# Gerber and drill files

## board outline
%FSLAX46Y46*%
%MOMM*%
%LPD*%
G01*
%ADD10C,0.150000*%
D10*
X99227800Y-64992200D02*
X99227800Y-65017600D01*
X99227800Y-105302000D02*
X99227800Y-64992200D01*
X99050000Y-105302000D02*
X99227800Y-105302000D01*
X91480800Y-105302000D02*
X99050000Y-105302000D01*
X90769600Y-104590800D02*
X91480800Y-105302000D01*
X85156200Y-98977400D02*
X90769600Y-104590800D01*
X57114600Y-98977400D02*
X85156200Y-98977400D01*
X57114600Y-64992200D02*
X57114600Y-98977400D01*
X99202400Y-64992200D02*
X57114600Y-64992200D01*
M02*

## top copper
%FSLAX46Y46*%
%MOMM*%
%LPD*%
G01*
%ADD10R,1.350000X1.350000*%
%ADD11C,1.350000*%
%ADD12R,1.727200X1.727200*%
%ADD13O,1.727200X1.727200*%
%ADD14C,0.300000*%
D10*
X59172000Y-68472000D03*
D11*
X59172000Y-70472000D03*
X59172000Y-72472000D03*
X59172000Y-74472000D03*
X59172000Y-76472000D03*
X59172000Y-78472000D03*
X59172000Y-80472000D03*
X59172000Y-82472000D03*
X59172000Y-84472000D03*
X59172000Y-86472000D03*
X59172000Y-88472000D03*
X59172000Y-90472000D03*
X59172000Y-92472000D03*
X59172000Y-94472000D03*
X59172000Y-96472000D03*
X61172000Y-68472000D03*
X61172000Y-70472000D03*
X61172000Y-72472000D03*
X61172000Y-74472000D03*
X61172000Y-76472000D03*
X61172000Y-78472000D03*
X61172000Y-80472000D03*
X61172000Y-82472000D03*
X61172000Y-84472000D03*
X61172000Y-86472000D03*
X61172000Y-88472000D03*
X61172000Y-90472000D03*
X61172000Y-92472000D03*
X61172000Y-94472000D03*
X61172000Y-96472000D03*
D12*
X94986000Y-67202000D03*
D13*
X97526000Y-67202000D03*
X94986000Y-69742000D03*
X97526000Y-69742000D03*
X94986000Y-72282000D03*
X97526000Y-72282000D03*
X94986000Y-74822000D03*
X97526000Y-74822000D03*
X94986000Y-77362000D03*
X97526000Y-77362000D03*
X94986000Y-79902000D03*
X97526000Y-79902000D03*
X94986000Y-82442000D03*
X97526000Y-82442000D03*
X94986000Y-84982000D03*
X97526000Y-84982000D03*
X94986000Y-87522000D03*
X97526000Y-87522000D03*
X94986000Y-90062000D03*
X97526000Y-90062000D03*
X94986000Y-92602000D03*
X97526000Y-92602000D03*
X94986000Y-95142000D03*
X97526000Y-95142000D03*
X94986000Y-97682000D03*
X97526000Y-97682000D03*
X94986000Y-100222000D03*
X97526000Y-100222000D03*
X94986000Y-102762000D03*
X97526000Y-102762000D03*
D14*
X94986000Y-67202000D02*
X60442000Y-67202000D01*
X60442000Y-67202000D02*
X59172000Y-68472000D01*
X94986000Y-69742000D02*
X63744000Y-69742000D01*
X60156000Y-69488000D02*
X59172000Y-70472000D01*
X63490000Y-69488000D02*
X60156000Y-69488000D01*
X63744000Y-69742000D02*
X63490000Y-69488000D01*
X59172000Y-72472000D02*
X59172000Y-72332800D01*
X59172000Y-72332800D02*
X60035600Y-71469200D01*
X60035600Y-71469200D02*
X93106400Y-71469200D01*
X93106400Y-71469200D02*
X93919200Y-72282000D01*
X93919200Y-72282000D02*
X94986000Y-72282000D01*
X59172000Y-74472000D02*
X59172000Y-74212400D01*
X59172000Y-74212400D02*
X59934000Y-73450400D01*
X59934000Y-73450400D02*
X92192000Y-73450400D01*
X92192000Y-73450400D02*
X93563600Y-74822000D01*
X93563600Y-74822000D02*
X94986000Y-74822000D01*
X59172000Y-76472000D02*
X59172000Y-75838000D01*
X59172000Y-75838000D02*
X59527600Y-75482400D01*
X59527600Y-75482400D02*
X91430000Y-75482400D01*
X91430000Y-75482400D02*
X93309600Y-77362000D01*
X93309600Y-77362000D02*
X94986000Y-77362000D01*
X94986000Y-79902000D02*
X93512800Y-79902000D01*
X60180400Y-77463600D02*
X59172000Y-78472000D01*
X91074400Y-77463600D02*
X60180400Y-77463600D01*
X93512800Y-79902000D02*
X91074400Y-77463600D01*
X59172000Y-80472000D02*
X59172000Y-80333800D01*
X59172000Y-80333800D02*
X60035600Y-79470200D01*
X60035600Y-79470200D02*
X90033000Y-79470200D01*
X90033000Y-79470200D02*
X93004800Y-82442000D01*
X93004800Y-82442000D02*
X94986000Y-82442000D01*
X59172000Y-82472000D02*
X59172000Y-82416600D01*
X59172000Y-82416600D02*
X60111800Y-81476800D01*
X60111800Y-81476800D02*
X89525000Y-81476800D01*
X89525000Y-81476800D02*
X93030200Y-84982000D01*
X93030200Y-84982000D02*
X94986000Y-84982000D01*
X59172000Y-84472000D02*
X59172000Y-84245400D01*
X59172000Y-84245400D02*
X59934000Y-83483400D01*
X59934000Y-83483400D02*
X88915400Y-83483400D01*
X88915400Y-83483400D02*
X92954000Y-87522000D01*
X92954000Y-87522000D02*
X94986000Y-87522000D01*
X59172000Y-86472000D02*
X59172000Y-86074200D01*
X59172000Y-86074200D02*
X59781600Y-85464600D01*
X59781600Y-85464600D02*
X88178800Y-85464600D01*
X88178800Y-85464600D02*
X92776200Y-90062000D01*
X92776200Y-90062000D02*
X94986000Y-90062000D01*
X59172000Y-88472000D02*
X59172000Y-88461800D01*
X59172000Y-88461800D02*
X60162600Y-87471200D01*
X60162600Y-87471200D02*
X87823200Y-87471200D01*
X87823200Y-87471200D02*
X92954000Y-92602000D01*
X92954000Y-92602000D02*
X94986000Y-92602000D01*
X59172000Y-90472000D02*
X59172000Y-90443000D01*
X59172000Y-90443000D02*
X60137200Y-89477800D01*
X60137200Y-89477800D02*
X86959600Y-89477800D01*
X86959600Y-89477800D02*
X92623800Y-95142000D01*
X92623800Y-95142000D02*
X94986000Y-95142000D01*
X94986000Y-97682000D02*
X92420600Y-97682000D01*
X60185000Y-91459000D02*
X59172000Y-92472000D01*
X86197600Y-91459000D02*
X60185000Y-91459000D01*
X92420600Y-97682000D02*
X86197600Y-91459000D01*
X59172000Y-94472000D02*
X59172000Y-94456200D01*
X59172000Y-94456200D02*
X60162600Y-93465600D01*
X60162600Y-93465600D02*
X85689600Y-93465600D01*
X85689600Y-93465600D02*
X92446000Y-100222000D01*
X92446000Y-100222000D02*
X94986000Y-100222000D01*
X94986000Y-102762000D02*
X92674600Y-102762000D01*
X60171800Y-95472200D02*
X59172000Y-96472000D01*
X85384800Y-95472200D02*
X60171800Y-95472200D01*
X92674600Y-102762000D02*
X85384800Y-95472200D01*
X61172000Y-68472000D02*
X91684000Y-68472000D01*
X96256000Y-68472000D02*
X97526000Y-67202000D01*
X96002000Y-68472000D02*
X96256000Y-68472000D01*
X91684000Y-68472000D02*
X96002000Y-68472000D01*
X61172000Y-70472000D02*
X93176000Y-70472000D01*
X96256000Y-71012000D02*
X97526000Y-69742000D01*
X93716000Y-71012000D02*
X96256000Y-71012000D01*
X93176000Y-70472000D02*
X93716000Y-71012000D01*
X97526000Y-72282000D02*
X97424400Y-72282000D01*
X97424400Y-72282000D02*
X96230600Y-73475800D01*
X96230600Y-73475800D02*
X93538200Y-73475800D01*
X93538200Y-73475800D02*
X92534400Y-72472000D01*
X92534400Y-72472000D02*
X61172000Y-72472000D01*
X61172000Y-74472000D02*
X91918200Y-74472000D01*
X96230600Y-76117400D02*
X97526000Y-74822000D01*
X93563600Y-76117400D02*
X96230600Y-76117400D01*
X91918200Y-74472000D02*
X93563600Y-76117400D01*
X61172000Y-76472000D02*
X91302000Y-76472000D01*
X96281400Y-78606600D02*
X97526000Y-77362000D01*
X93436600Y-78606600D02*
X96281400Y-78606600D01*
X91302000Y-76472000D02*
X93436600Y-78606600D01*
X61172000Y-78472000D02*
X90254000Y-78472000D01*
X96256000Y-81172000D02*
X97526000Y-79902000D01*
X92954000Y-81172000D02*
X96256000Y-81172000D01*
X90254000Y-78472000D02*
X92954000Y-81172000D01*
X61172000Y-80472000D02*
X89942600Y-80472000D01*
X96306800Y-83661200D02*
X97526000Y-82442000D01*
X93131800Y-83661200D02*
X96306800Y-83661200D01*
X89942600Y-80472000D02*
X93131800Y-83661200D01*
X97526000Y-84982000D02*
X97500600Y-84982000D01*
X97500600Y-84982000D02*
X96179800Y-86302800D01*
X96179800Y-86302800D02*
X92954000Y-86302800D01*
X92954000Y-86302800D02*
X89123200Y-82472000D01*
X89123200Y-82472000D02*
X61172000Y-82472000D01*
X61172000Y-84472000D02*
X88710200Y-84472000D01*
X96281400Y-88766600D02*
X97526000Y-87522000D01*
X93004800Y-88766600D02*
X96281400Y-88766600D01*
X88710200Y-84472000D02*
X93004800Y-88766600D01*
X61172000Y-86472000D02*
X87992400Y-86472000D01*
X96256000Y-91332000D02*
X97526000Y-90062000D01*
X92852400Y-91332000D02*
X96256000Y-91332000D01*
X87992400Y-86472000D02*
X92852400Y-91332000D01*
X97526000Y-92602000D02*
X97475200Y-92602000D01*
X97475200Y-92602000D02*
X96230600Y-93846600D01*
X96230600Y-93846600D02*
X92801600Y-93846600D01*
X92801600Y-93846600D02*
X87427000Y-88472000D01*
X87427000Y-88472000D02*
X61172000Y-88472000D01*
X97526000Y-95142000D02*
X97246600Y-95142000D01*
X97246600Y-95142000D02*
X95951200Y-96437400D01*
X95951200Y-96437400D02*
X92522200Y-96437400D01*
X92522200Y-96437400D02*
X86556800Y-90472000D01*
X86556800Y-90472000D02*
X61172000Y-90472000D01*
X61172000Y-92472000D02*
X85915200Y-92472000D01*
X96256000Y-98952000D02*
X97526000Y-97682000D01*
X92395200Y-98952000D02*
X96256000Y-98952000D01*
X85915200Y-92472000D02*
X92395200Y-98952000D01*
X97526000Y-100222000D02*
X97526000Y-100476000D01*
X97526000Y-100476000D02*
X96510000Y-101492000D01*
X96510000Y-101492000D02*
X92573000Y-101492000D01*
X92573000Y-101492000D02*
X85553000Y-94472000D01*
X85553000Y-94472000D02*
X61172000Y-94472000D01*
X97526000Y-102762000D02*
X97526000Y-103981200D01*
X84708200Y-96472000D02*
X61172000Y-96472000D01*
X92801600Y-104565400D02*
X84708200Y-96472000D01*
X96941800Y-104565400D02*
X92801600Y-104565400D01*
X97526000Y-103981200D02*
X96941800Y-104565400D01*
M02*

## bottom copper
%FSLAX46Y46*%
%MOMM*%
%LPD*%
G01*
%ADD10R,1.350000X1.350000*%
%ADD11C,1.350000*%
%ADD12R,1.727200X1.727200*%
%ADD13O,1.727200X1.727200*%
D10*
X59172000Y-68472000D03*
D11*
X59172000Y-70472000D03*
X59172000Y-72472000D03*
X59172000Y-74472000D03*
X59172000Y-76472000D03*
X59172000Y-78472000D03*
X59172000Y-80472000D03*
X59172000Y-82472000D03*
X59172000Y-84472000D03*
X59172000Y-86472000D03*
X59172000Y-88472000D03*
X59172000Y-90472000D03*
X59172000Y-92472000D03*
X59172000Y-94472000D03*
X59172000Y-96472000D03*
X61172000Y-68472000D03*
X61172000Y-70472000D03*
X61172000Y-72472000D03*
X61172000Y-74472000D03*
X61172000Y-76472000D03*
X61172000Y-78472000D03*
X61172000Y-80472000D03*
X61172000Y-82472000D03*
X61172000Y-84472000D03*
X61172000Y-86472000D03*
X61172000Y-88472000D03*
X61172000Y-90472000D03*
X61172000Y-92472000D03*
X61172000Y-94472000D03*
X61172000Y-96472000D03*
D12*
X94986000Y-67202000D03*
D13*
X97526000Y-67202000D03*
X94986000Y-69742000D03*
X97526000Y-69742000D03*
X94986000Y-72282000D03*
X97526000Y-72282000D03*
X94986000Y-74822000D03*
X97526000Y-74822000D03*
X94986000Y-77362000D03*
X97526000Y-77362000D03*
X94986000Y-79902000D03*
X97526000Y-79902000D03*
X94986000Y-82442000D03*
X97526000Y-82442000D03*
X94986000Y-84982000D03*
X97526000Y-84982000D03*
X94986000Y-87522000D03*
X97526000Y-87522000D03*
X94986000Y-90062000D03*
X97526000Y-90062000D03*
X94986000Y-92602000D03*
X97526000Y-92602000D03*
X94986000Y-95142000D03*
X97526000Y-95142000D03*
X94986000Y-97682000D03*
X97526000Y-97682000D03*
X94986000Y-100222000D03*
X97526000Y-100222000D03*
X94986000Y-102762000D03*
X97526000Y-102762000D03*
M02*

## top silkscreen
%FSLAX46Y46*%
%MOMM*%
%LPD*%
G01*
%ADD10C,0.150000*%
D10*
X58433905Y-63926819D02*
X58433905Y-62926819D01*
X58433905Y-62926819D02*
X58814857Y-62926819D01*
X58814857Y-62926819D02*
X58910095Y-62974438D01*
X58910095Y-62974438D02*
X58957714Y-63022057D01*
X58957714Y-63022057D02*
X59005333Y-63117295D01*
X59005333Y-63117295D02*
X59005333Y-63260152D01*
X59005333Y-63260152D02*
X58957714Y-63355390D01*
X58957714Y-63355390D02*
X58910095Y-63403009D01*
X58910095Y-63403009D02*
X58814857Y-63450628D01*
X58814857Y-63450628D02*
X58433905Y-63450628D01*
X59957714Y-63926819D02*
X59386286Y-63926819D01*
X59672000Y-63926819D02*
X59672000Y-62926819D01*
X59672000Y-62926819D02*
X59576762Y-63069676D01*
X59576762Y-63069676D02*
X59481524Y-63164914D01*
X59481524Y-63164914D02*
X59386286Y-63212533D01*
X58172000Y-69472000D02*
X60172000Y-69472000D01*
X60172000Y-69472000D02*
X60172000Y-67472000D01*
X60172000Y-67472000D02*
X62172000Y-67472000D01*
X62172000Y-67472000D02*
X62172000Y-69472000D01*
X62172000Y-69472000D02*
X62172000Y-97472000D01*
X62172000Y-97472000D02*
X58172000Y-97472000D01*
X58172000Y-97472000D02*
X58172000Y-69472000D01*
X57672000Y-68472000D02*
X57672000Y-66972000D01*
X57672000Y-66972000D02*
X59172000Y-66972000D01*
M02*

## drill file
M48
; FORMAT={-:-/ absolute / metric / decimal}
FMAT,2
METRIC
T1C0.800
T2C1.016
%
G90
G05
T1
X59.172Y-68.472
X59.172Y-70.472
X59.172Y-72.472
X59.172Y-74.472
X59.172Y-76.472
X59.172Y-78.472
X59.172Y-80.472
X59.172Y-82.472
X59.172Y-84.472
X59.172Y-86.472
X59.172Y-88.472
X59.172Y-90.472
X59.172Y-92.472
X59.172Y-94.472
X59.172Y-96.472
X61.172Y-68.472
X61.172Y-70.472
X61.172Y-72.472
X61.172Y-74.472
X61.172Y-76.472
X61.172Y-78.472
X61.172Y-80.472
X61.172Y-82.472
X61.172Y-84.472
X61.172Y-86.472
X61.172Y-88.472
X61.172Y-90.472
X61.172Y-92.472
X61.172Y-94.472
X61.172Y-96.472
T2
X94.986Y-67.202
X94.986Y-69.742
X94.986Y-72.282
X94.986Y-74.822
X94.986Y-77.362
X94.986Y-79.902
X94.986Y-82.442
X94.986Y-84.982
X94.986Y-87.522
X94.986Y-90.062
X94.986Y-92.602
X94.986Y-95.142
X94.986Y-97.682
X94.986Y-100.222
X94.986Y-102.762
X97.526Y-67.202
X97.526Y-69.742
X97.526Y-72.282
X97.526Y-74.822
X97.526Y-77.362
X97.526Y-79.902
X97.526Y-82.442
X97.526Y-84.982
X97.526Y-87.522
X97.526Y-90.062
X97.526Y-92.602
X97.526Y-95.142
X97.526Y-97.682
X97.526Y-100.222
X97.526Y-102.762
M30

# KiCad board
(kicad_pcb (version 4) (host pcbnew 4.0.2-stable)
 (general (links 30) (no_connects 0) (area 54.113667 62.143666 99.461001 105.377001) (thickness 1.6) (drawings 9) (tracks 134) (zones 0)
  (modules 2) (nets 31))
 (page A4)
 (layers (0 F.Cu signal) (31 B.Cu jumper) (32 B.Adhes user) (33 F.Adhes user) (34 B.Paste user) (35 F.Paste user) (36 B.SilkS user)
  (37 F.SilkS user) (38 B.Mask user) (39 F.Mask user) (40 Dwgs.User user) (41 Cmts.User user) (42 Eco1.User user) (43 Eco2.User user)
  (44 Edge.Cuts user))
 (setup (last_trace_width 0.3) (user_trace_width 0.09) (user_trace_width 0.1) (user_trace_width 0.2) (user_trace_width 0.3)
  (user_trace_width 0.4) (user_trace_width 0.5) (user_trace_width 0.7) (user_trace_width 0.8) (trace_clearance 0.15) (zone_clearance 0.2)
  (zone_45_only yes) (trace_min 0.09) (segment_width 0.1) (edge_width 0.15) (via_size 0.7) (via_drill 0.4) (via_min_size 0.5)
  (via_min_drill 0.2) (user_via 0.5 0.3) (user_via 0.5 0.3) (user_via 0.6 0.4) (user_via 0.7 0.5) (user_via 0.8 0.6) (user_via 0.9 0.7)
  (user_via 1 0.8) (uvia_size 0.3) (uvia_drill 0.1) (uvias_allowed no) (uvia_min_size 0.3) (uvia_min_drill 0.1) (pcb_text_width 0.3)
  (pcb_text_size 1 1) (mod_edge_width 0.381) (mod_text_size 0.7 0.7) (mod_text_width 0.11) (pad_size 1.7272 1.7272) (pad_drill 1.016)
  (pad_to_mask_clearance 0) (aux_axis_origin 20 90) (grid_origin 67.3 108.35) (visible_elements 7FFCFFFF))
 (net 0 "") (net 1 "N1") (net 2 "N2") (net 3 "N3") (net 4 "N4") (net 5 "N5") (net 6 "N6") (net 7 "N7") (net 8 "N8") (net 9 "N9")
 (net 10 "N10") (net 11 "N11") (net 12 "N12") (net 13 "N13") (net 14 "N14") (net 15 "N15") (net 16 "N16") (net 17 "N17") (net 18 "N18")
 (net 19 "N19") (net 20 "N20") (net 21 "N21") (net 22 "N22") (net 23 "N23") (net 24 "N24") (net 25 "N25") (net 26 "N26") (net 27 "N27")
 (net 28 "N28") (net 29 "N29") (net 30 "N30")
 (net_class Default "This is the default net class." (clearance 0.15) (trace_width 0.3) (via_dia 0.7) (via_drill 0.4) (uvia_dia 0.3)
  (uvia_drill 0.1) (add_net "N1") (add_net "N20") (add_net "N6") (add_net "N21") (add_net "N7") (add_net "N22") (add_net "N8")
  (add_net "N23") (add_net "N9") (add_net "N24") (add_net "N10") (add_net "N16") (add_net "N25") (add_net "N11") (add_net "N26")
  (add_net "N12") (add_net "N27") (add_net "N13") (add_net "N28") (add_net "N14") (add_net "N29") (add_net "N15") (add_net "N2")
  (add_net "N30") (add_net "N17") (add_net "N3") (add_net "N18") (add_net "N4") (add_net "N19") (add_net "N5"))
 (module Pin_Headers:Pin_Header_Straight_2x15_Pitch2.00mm (layer F.Cu) (at 59.172 68.472)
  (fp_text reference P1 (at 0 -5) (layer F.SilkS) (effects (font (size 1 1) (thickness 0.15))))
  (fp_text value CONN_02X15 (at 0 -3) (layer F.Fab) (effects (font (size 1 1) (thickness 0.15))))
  (fp_line (start -1 1) (end 1 1) (layer F.SilkS) (width 0.15))
  (fp_line (start 1 1) (end 1 -1) (layer F.SilkS) (width 0.15))
  (fp_line (start 1 -1) (end 3 -1) (layer F.SilkS) (width 0.15))
  (fp_line (start 3 -1) (end 3 1) (layer F.SilkS) (width 0.15))
  (fp_line (start 3 1) (end 3 29) (layer F.SilkS) (width 0.15))
  (fp_line (start 3 29) (end -1 29) (layer F.SilkS) (width 0.15))
  (fp_line (start -1 29) (end -1 1) (layer F.SilkS) (width 0.15))
  (fp_line (start -1.5 0) (end -1.5 -1.5) (layer F.SilkS) (width 0.15))
  (fp_line (start -1.5 -1.5) (end 0 -1.5) (layer F.SilkS) (width 0.15))
  (pad 1 thru_hole rect (at 0 0) (size 1.35 1.35) (drill 0.8) (layers *.Cu *.Mask) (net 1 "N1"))
  (pad 3 thru_hole circle (at 0 2) (size 1.35 1.35) (drill 0.8) (layers *.Cu *.Mask) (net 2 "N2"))
  (pad 5 thru_hole circle (at 0 4) (size 1.35 1.35) (drill 0.8) (layers *.Cu *.Mask) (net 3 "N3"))
  (pad 7 thru_hole circle (at 0 6) (size 1.35 1.35) (drill 0.8) (layers *.Cu *.Mask) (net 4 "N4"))
  (pad 9 thru_hole circle (at 0 8) (size 1.35 1.35) (drill 0.8) (layers *.Cu *.Mask) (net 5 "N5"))
  (pad 11 thru_hole circle (at 0 10) (size 1.35 1.35) (drill 0.8) (layers *.Cu *.Mask) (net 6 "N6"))
  (pad 13 thru_hole circle (at 0 12) (size 1.35 1.35) (drill 0.8) (layers *.Cu *.Mask) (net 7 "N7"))
  (pad 15 thru_hole circle (at 0 14) (size 1.35 1.35) (drill 0.8) (layers *.Cu *.Mask) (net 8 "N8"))
  (pad 17 thru_hole circle (at 0 16) (size 1.35 1.35) (drill 0.8) (layers *.Cu *.Mask) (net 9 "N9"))
  (pad 19 thru_hole circle (at 0 18) (size 1.35 1.35) (drill 0.8) (layers *.Cu *.Mask) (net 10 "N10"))
  (pad 21 thru_hole circle (at 0 20) (size 1.35 1.35) (drill 0.8) (layers *.Cu *.Mask) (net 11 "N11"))
  (pad 23 thru_hole circle (at 0 22) (size 1.35 1.35) (drill 0.8) (layers *.Cu *.Mask) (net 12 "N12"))
  (pad 25 thru_hole circle (at 0 24) (size 1.35 1.35) (drill 0.8) (layers *.Cu *.Mask) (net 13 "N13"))
  (pad 27 thru_hole circle (at 0 26) (size 1.35 1.35) (drill 0.8) (layers *.Cu *.Mask) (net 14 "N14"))
  (pad 29 thru_hole circle (at 0 28) (size 1.35 1.35) (drill 0.8) (layers *.Cu *.Mask) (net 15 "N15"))
  (pad 2 thru_hole circle (at 2 0) (size 1.35 1.35) (drill 0.8) (layers *.Cu *.Mask) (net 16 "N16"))
  (pad 4 thru_hole circle (at 2 2) (size 1.35 1.35) (drill 0.8) (layers *.Cu *.Mask) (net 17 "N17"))
  (pad 6 thru_hole circle (at 2 4) (size 1.35 1.35) (drill 0.8) (layers *.Cu *.Mask) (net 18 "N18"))
  (pad 8 thru_hole circle (at 2 6) (size 1.35 1.35) (drill 0.8) (layers *.Cu *.Mask) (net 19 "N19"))
  (pad 10 thru_hole circle (at 2 8) (size 1.35 1.35) (drill 0.8) (layers *.Cu *.Mask) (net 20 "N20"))
  (pad 12 thru_hole circle (at 2 10) (size 1.35 1.35) (drill 0.8) (layers *.Cu *.Mask) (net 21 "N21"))
  (pad 14 thru_hole circle (at 2 12) (size 1.35 1.35) (drill 0.8) (layers *.Cu *.Mask) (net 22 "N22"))
  (pad 16 thru_hole circle (at 2 14) (size 1.35 1.35) (drill 0.8) (layers *.Cu *.Mask) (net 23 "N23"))
  (pad 18 thru_hole circle (at 2 16) (size 1.35 1.35) (drill 0.8) (layers *.Cu *.Mask) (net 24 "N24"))
  (pad 20 thru_hole circle (at 2 18) (size 1.35 1.35) (drill 0.8) (layers *.Cu *.Mask) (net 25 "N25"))
  (pad 22 thru_hole circle (at 2 20) (size 1.35 1.35) (drill 0.8) (layers *.Cu *.Mask) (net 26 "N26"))
  (pad 24 thru_hole circle (at 2 22) (size 1.35 1.35) (drill 0.8) (layers *.Cu *.Mask) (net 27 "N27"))
  (pad 26 thru_hole circle (at 2 24) (size 1.35 1.35) (drill 0.8) (layers *.Cu *.Mask) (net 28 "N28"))
  (pad 28 thru_hole circle (at 2 26) (size 1.35 1.35) (drill 0.8) (layers *.Cu *.Mask) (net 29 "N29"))
  (pad 30 thru_hole circle (at 2 28) (size 1.35 1.35) (drill 0.8) (layers *.Cu *.Mask) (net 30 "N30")))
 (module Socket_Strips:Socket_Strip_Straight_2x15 (layer B.Cu) (at 94.986 67.202 270)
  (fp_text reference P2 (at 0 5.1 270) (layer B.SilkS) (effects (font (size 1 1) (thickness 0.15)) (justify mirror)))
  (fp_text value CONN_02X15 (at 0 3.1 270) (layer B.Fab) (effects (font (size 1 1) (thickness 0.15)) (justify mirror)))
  (pad 1 thru_hole rect (at 0 0 270) (size 1.7272 1.7272) (drill 1.016) (layers *.Cu *.Mask B.SilkS) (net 1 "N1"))
  (pad 2 thru_hole oval (at 0 -2.54 270) (size 1.7272 1.7272) (drill 1.016) (layers *.Cu *.Mask B.SilkS) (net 16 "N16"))
  (pad 3 thru_hole oval (at 2.54 0 270) (size 1.7272 1.7272) (drill 1.016) (layers *.Cu *.Mask B.SilkS) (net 2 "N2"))
  (pad 4 thru_hole oval (at 2.54 -2.54 270) (size 1.7272 1.7272) (drill 1.016) (layers *.Cu *.Mask B.SilkS) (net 17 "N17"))
  (pad 5 thru_hole oval (at 5.08 0 270) (size 1.7272 1.7272) (drill 1.016) (layers *.Cu *.Mask B.SilkS) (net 3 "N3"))
  (pad 6 thru_hole oval (at 5.08 -2.54 270) (size 1.7272 1.7272) (drill 1.016) (layers *.Cu *.Mask B.SilkS) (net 18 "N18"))
  (pad 7 thru_hole oval (at 7.62 0 270) (size 1.7272 1.7272) (drill 1.016) (layers *.Cu *.Mask B.SilkS) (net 4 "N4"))
  (pad 8 thru_hole oval (at 7.62 -2.54 270) (size 1.7272 1.7272) (drill 1.016) (layers *.Cu *.Mask B.SilkS) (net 19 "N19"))
  (pad 9 thru_hole oval (at 10.16 0 270) (size 1.7272 1.7272) (drill 1.016) (layers *.Cu *.Mask B.SilkS) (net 5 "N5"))
  (pad 10 thru_hole oval (at 10.16 -2.54 270) (size 1.7272 1.7272) (drill 1.016) (layers *.Cu *.Mask B.SilkS) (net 20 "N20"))
  (pad 11 thru_hole oval (at 12.7 0 270) (size 1.7272 1.7272) (drill 1.016) (layers *.Cu *.Mask B.SilkS) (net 6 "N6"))
  (pad 12 thru_hole oval (at 12.7 -2.54 270) (size 1.7272 1.7272) (drill 1.016) (layers *.Cu *.Mask B.SilkS) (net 21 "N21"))
  (pad 13 thru_hole oval (at 15.24 0 270) (size 1.7272 1.7272) (drill 1.016) (layers *.Cu *.Mask B.SilkS) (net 7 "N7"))
  (pad 14 thru_hole oval (at 15.24 -2.54 270) (size 1.7272 1.7272) (drill 1.016) (layers *.Cu *.Mask B.SilkS) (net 22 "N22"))
  (pad 15 thru_hole oval (at 17.78 0 270) (size 1.7272 1.7272) (drill 1.016) (layers *.Cu *.Mask B.SilkS) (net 8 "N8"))
  (pad 16 thru_hole oval (at 17.78 -2.54 270) (size 1.7272 1.7272) (drill 1.016) (layers *.Cu *.Mask B.SilkS) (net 23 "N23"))
  (pad 17 thru_hole oval (at 20.32 0 270) (size 1.7272 1.7272) (drill 1.016) (layers *.Cu *.Mask B.SilkS) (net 9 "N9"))
  (pad 18 thru_hole oval (at 20.32 -2.54 270) (size 1.7272 1.7272) (drill 1.016) (layers *.Cu *.Mask B.SilkS) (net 24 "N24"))
  (pad 19 thru_hole oval (at 22.86 0 270) (size 1.7272 1.7272) (drill 1.016) (layers *.Cu *.Mask B.SilkS) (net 10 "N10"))
  (pad 20 thru_hole oval (at 22.86 -2.54 270) (size 1.7272 1.7272) (drill 1.016) (layers *.Cu *.Mask B.SilkS) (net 25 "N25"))
  (pad 21 thru_hole oval (at 25.4 0 270) (size 1.7272 1.7272) (drill 1.016) (layers *.Cu *.Mask B.SilkS) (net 11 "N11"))
  (pad 22 thru_hole oval (at 25.4 -2.54 270) (size 1.7272 1.7272) (drill 1.016) (layers *.Cu *.Mask B.SilkS) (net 26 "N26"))
  (pad 23 thru_hole oval (at 27.94 0 270) (size 1.7272 1.7272) (drill 1.016) (layers *.Cu *.Mask B.SilkS) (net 12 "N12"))
  (pad 24 thru_hole oval (at 27.94 -2.54 270) (size 1.7272 1.7272) (drill 1.016) (layers *.Cu *.Mask B.SilkS) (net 27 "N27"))
  (pad 25 thru_hole oval (at 30.48 0 270) (size 1.7272 1.7272) (drill 1.016) (layers *.Cu *.Mask B.SilkS) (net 13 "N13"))
  (pad 26 thru_hole oval (at 30.48 -2.54 270) (size 1.7272 1.7272) (drill 1.016) (layers *.Cu *.Mask B.SilkS) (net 28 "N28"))
  (pad 27 thru_hole oval (at 33.02 0 270) (size 1.7272 1.7272) (drill 1.016) (layers *.Cu *.Mask B.SilkS) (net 14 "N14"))
  (pad 28 thru_hole oval (at 33.02 -2.54 270) (size 1.7272 1.7272) (drill 1.016) (layers *.Cu *.Mask B.SilkS) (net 29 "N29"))
  (pad 29 thru_hole oval (at 35.56 0 270) (size 1.7272 1.7272) (drill 1.016) (layers *.Cu *.Mask B.SilkS) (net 15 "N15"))
  (pad 30 thru_hole oval (at 35.56 -2.54 270) (size 1.7272 1.7272) (drill 1.016) (layers *.Cu *.Mask B.SilkS) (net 30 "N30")))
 (gr_line (start 99.2278 64.9922) (end 99.2278 65.0176) (angle 90) (layer Edge.Cuts) (width 0.15))
 (gr_line (start 99.2278 105.302) (end 99.2278 64.9922) (angle 90) (layer Edge.Cuts) (width 0.15))
 (gr_line (start 99.05 105.302) (end 99.2278 105.302) (angle 90) (layer Edge.Cuts) (width 0.15))
 (gr_line (start 91.4808 105.302) (end 99.05 105.302) (angle 90) (layer Edge.Cuts) (width 0.15))
 (gr_line (start 90.7696 104.5908) (end 91.4808 105.302) (angle 90) (layer Edge.Cuts) (width 0.15))
 (gr_line (start 85.1562 98.9774) (end 90.7696 104.5908) (angle 90) (layer Edge.Cuts) (width 0.15))
 (gr_line (start 57.1146 98.9774) (end 85.1562 98.9774) (angle 90) (layer Edge.Cuts) (width 0.15))
 (gr_line (start 57.1146 64.9922) (end 57.1146 98.9774) (angle 90) (layer Edge.Cuts) (width 0.15))
 (gr_line (start 99.2024 64.9922) (end 57.1146 64.9922) (angle 90) (layer Edge.Cuts) (width 0.15))
 (segment (start 94.986 67.202) (end 60.442 67.202) (width 0.3) (layer F.Cu) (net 1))
 (segment (start 60.442 67.202) (end 59.172 68.472) (width 0.3) (layer F.Cu) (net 1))
 (segment (start 94.986 69.742) (end 63.744 69.742) (width 0.3) (layer F.Cu) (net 2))
 (segment (start 60.156 69.488) (end 59.172 70.472) (width 0.3) (layer F.Cu) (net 2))
 (segment (start 63.49 69.488) (end 60.156 69.488) (width 0.3) (layer F.Cu) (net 2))
 (segment (start 63.744 69.742) (end 63.49 69.488) (width 0.3) (layer F.Cu) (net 2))
 (segment (start 59.172 72.472) (end 59.172 72.3328) (width 0.3) (layer F.Cu) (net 3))
 (segment (start 59.172 72.3328) (end 60.0356 71.4692) (width 0.3) (layer F.Cu) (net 3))
 (segment (start 60.0356 71.4692) (end 93.1064 71.4692) (width 0.3) (layer F.Cu) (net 3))
 (segment (start 93.1064 71.4692) (end 93.9192 72.282) (width 0.3) (layer F.Cu) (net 3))
 (segment (start 93.9192 72.282) (end 94.986 72.282) (width 0.3) (layer F.Cu) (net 3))
 (segment (start 59.172 74.472) (end 59.172 74.2124) (width 0.3) (layer F.Cu) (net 4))
 (segment (start 59.172 74.2124) (end 59.934 73.4504) (width 0.3) (layer F.Cu) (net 4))
 (segment (start 59.934 73.4504) (end 92.192 73.4504) (width 0.3) (layer F.Cu) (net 4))
 (segment (start 92.192 73.4504) (end 93.5636 74.822) (width 0.3) (layer F.Cu) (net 4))
 (segment (start 93.5636 74.822) (end 94.986 74.822) (width 0.3) (layer F.Cu) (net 4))
 (segment (start 59.172 76.472) (end 59.172 75.838) (width 0.3) (layer F.Cu) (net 5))
 (segment (start 59.172 75.838) (end 59.5276 75.4824) (width 0.3) (layer F.Cu) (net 5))
 (segment (start 59.5276 75.4824) (end 91.43 75.4824) (width 0.3) (layer F.Cu) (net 5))
 (segment (start 91.43 75.4824) (end 93.3096 77.362) (width 0.3) (layer F.Cu) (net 5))
 (segment (start 93.3096 77.362) (end 94.986 77.362) (width 0.3) (layer F.Cu) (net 5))
 (segment (start 94.986 79.902) (end 93.5128 79.902) (width 0.3) (layer F.Cu) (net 6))
 (segment (start 60.1804 77.4636) (end 59.172 78.472) (width 0.3) (layer F.Cu) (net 6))
 (segment (start 91.0744 77.4636) (end 60.1804 77.4636) (width 0.3) (layer F.Cu) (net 6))
 (segment (start 93.5128 79.902) (end 91.0744 77.4636) (width 0.3) (layer F.Cu) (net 6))
 (segment (start 59.172 80.472) (end 59.172 80.3338) (width 0.3) (layer F.Cu) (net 7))
 (segment (start 59.172 80.3338) (end 60.0356 79.4702) (width 0.3) (layer F.Cu) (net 7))
 (segment (start 60.0356 79.4702) (end 90.033 79.4702) (width 0.3) (layer F.Cu) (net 7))
 (segment (start 90.033 79.4702) (end 93.0048 82.442) (width 0.3) (layer F.Cu) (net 7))
 (segment (start 93.0048 82.442) (end 94.986 82.442) (width 0.3) (layer F.Cu) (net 7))
 (segment (start 59.172 82.472) (end 59.172 82.4166) (width 0.3) (layer F.Cu) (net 8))
 (segment (start 59.172 82.4166) (end 60.1118 81.4768) (width 0.3) (layer F.Cu) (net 8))
 (segment (start 60.1118 81.4768) (end 89.525 81.4768) (width 0.3) (layer F.Cu) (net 8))
 (segment (start 89.525 81.4768) (end 93.0302 84.982) (width 0.3) (layer F.Cu) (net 8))
 (segment (start 93.0302 84.982) (end 94.986 84.982) (width 0.3) (layer F.Cu) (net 8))
 (segment (start 59.172 84.472) (end 59.172 84.2454) (width 0.3) (layer F.Cu) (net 9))
 (segment (start 59.172 84.2454) (end 59.934 83.4834) (width 0.3) (layer F.Cu) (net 9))
 (segment (start 59.934 83.4834) (end 88.9154 83.4834) (width 0.3) (layer F.Cu) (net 9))
 (segment (start 88.9154 83.4834) (end 92.954 87.522) (width 0.3) (layer F.Cu) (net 9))
 (segment (start 92.954 87.522) (end 94.986 87.522) (width 0.3) (layer F.Cu) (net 9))
 (segment (start 59.172 86.472) (end 59.172 86.0742) (width 0.3) (layer F.Cu) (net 10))
 (segment (start 59.172 86.0742) (end 59.7816 85.4646) (width 0.3) (layer F.Cu) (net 10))
 (segment (start 59.7816 85.4646) (end 88.1788 85.4646) (width 0.3) (layer F.Cu) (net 10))
 (segment (start 88.1788 85.4646) (end 92.7762 90.062) (width 0.3) (layer F.Cu) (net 10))
 (segment (start 92.7762 90.062) (end 94.986 90.062) (width 0.3) (layer F.Cu) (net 10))
 (segment (start 59.172 88.472) (end 59.172 88.4618) (width 0.3) (layer F.Cu) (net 11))
 (segment (start 59.172 88.4618) (end 60.1626 87.4712) (width 0.3) (layer F.Cu) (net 11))
 (segment (start 60.1626 87.4712) (end 87.8232 87.4712) (width 0.3) (layer F.Cu) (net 11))
 (segment (start 87.8232 87.4712) (end 92.954 92.602) (width 0.3) (layer F.Cu) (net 11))
 (segment (start 92.954 92.602) (end 94.986 92.602) (width 0.3) (layer F.Cu) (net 11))
 (segment (start 59.172 90.472) (end 59.172 90.443) (width 0.3) (layer F.Cu) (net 12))
 (segment (start 59.172 90.443) (end 60.1372 89.4778) (width 0.3) (layer F.Cu) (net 12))
 (segment (start 60.1372 89.4778) (end 86.9596 89.4778) (width 0.3) (layer F.Cu) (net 12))
 (segment (start 86.9596 89.4778) (end 92.6238 95.142) (width 0.3) (layer F.Cu) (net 12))
 (segment (start 92.6238 95.142) (end 94.986 95.142) (width 0.3) (layer F.Cu) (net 12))
 (segment (start 94.986 97.682) (end 92.4206 97.682) (width 0.3) (layer F.Cu) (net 13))
 (segment (start 60.185 91.459) (end 59.172 92.472) (width 0.3) (layer F.Cu) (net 13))
 (segment (start 86.1976 91.459) (end 60.185 91.459) (width 0.3) (layer F.Cu) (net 13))
 (segment (start 92.4206 97.682) (end 86.1976 91.459) (width 0.3) (layer F.Cu) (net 13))
 (segment (start 59.172 94.472) (end 59.172 94.4562) (width 0.3) (layer F.Cu) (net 14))
 (segment (start 59.172 94.4562) (end 60.1626 93.4656) (width 0.3) (layer F.Cu) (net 14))
 (segment (start 60.1626 93.4656) (end 85.6896 93.4656) (width 0.3) (layer F.Cu) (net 14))
 (segment (start 85.6896 93.4656) (end 92.446 100.222) (width 0.3) (layer F.Cu) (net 14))
 (segment (start 92.446 100.222) (end 94.986 100.222) (width 0.3) (layer F.Cu) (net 14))
 (segment (start 94.986 102.762) (end 92.6746 102.762) (width 0.3) (layer F.Cu) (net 15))
 (segment (start 60.1718 95.4722) (end 59.172 96.472) (width 0.3) (layer F.Cu) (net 15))
 (segment (start 85.3848 95.4722) (end 60.1718 95.4722) (width 0.3) (layer F.Cu) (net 15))
 (segment (start 92.6746 102.762) (end 85.3848 95.4722) (width 0.3) (layer F.Cu) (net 15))
 (segment (start 61.172 68.472) (end 91.684 68.472) (width 0.3) (layer F.Cu) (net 16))
 (segment (start 96.256 68.472) (end 97.526 67.202) (width 0.3) (layer F.Cu) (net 16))
 (segment (start 96.002 68.472) (end 96.256 68.472) (width 0.3) (layer F.Cu) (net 16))
 (segment (start 91.684 68.472) (end 96.002 68.472) (width 0.3) (layer F.Cu) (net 16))
 (segment (start 61.172 70.472) (end 93.176 70.472) (width 0.3) (layer F.Cu) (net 17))
 (segment (start 96.256 71.012) (end 97.526 69.742) (width 0.3) (layer F.Cu) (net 17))
 (segment (start 93.716 71.012) (end 96.256 71.012) (width 0.3) (layer F.Cu) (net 17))
 (segment (start 93.176 70.472) (end 93.716 71.012) (width 0.3) (layer F.Cu) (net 17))
 (segment (start 97.526 72.282) (end 97.4244 72.282) (width 0.3) (layer F.Cu) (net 18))
 (segment (start 97.4244 72.282) (end 96.2306 73.4758) (width 0.3) (layer F.Cu) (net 18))
 (segment (start 96.2306 73.4758) (end 93.5382 73.4758) (width 0.3) (layer F.Cu) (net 18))
 (segment (start 93.5382 73.4758) (end 92.5344 72.472) (width 0.3) (layer F.Cu) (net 18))
 (segment (start 92.5344 72.472) (end 61.172 72.472) (width 0.3) (layer F.Cu) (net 18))
 (segment (start 61.172 74.472) (end 91.9182 74.472) (width 0.3) (layer F.Cu) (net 19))
 (segment (start 96.2306 76.1174) (end 97.526 74.822) (width 0.3) (layer F.Cu) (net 19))
 (segment (start 93.5636 76.1174) (end 96.2306 76.1174) (width 0.3) (layer F.Cu) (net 19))
 (segment (start 91.9182 74.472) (end 93.5636 76.1174) (width 0.3) (layer F.Cu) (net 19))
 (segment (start 61.172 76.472) (end 91.302 76.472) (width 0.3) (layer F.Cu) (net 20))
 (segment (start 96.2814 78.6066) (end 97.526 77.362) (width 0.3) (layer F.Cu) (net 20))
 (segment (start 93.4366 78.6066) (end 96.2814 78.6066) (width 0.3) (layer F.Cu) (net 20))
 (segment (start 91.302 76.472) (end 93.4366 78.6066) (width 0.3) (layer F.Cu) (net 20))
 (segment (start 61.172 78.472) (end 90.254 78.472) (width 0.3) (layer F.Cu) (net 21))
 (segment (start 96.256 81.172) (end 97.526 79.902) (width 0.3) (layer F.Cu) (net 21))
 (segment (start 92.954 81.172) (end 96.256 81.172) (width 0.3) (layer F.Cu) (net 21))
 (segment (start 90.254 78.472) (end 92.954 81.172) (width 0.3) (layer F.Cu) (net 21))
 (segment (start 61.172 80.472) (end 89.9426 80.472) (width 0.3) (layer F.Cu) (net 22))
 (segment (start 96.3068 83.6612) (end 97.526 82.442) (width 0.3) (layer F.Cu) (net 22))
 (segment (start 93.1318 83.6612) (end 96.3068 83.6612) (width 0.3) (layer F.Cu) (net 22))
 (segment (start 89.9426 80.472) (end 93.1318 83.6612) (width 0.3) (layer F.Cu) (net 22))
 (segment (start 97.526 84.982) (end 97.5006 84.982) (width 0.3) (layer F.Cu) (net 23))
 (segment (start 97.5006 84.982) (end 96.1798 86.3028) (width 0.3) (layer F.Cu) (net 23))
 (segment (start 96.1798 86.3028) (end 92.954 86.3028) (width 0.3) (layer F.Cu) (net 23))
 (segment (start 92.954 86.3028) (end 89.1232 82.472) (width 0.3) (layer F.Cu) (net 23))
 (segment (start 89.1232 82.472) (end 61.172 82.472) (width 0.3) (layer F.Cu) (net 23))
 (segment (start 61.172 84.472) (end 88.7102 84.472) (width 0.3) (layer F.Cu) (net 24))
 (segment (start 96.2814 88.7666) (end 97.526 87.522) (width 0.3) (layer F.Cu) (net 24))
 (segment (start 93.0048 88.7666) (end 96.2814 88.7666) (width 0.3) (layer F.Cu) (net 24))
 (segment (start 88.7102 84.472) (end 93.0048 88.7666) (width 0.3) (layer F.Cu) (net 24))
 (segment (start 61.172 86.472) (end 87.9924 86.472) (width 0.3) (layer F.Cu) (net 25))
 (segment (start 96.256 91.332) (end 97.526 90.062) (width 0.3) (layer F.Cu) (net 25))
 (segment (start 92.8524 91.332) (end 96.256 91.332) (width 0.3) (layer F.Cu) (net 25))
 (segment (start 87.9924 86.472) (end 92.8524 91.332) (width 0.3) (layer F.Cu) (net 25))
 (segment (start 97.526 92.602) (end 97.4752 92.602) (width 0.3) (layer F.Cu) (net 26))
 (segment (start 97.4752 92.602) (end 96.2306 93.8466) (width 0.3) (layer F.Cu) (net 26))
 (segment (start 96.2306 93.8466) (end 92.8016 93.8466) (width 0.3) (layer F.Cu) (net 26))
 (segment (start 92.8016 93.8466) (end 87.427 88.472) (width 0.3) (layer F.Cu) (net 26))
 (segment (start 87.427 88.472) (end 61.172 88.472) (width 0.3) (layer F.Cu) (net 26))
 (segment (start 97.526 95.142) (end 97.2466 95.142) (width 0.3) (layer F.Cu) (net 27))
 (segment (start 97.2466 95.142) (end 95.9512 96.4374) (width 0.3) (layer F.Cu) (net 27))
 (segment (start 95.9512 96.4374) (end 92.5222 96.4374) (width 0.3) (layer F.Cu) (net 27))
 (segment (start 92.5222 96.4374) (end 86.5568 90.472) (width 0.3) (layer F.Cu) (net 27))
 (segment (start 86.5568 90.472) (end 61.172 90.472) (width 0.3) (layer F.Cu) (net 27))
 (segment (start 61.172 92.472) (end 85.9152 92.472) (width 0.3) (layer F.Cu) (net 28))
 (segment (start 96.256 98.952) (end 97.526 97.682) (width 0.3) (layer F.Cu) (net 28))
 (segment (start 92.3952 98.952) (end 96.256 98.952) (width 0.3) (layer F.Cu) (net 28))
 (segment (start 85.9152 92.472) (end 92.3952 98.952) (width 0.3) (layer F.Cu) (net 28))
 (segment (start 97.526 100.222) (end 97.526 100.476) (width 0.3) (layer F.Cu) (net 29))
 (segment (start 97.526 100.476) (end 96.51 101.492) (width 0.3) (layer F.Cu) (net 29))
 (segment (start 96.51 101.492) (end 92.573 101.492) (width 0.3) (layer F.Cu) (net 29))
 (segment (start 92.573 101.492) (end 85.553 94.472) (width 0.3) (layer F.Cu) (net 29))
 (segment (start 85.553 94.472) (end 61.172 94.472) (width 0.3) (layer F.Cu) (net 29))
 (segment (start 97.526 102.762) (end 97.526 103.9812) (width 0.3) (layer F.Cu) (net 30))
 (segment (start 84.7082 96.472) (end 61.172 96.472) (width 0.3) (layer F.Cu) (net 30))
 (segment (start 92.8016 104.5654) (end 84.7082 96.472) (width 0.3) (layer F.Cu) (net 30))
 (segment (start 96.9418 104.5654) (end 92.8016 104.5654) (width 0.3) (layer F.Cu) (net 30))
 (segment (start 97.526 103.9812) (end 96.9418 104.5654) (width 0.3) (layer F.Cu) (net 30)))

